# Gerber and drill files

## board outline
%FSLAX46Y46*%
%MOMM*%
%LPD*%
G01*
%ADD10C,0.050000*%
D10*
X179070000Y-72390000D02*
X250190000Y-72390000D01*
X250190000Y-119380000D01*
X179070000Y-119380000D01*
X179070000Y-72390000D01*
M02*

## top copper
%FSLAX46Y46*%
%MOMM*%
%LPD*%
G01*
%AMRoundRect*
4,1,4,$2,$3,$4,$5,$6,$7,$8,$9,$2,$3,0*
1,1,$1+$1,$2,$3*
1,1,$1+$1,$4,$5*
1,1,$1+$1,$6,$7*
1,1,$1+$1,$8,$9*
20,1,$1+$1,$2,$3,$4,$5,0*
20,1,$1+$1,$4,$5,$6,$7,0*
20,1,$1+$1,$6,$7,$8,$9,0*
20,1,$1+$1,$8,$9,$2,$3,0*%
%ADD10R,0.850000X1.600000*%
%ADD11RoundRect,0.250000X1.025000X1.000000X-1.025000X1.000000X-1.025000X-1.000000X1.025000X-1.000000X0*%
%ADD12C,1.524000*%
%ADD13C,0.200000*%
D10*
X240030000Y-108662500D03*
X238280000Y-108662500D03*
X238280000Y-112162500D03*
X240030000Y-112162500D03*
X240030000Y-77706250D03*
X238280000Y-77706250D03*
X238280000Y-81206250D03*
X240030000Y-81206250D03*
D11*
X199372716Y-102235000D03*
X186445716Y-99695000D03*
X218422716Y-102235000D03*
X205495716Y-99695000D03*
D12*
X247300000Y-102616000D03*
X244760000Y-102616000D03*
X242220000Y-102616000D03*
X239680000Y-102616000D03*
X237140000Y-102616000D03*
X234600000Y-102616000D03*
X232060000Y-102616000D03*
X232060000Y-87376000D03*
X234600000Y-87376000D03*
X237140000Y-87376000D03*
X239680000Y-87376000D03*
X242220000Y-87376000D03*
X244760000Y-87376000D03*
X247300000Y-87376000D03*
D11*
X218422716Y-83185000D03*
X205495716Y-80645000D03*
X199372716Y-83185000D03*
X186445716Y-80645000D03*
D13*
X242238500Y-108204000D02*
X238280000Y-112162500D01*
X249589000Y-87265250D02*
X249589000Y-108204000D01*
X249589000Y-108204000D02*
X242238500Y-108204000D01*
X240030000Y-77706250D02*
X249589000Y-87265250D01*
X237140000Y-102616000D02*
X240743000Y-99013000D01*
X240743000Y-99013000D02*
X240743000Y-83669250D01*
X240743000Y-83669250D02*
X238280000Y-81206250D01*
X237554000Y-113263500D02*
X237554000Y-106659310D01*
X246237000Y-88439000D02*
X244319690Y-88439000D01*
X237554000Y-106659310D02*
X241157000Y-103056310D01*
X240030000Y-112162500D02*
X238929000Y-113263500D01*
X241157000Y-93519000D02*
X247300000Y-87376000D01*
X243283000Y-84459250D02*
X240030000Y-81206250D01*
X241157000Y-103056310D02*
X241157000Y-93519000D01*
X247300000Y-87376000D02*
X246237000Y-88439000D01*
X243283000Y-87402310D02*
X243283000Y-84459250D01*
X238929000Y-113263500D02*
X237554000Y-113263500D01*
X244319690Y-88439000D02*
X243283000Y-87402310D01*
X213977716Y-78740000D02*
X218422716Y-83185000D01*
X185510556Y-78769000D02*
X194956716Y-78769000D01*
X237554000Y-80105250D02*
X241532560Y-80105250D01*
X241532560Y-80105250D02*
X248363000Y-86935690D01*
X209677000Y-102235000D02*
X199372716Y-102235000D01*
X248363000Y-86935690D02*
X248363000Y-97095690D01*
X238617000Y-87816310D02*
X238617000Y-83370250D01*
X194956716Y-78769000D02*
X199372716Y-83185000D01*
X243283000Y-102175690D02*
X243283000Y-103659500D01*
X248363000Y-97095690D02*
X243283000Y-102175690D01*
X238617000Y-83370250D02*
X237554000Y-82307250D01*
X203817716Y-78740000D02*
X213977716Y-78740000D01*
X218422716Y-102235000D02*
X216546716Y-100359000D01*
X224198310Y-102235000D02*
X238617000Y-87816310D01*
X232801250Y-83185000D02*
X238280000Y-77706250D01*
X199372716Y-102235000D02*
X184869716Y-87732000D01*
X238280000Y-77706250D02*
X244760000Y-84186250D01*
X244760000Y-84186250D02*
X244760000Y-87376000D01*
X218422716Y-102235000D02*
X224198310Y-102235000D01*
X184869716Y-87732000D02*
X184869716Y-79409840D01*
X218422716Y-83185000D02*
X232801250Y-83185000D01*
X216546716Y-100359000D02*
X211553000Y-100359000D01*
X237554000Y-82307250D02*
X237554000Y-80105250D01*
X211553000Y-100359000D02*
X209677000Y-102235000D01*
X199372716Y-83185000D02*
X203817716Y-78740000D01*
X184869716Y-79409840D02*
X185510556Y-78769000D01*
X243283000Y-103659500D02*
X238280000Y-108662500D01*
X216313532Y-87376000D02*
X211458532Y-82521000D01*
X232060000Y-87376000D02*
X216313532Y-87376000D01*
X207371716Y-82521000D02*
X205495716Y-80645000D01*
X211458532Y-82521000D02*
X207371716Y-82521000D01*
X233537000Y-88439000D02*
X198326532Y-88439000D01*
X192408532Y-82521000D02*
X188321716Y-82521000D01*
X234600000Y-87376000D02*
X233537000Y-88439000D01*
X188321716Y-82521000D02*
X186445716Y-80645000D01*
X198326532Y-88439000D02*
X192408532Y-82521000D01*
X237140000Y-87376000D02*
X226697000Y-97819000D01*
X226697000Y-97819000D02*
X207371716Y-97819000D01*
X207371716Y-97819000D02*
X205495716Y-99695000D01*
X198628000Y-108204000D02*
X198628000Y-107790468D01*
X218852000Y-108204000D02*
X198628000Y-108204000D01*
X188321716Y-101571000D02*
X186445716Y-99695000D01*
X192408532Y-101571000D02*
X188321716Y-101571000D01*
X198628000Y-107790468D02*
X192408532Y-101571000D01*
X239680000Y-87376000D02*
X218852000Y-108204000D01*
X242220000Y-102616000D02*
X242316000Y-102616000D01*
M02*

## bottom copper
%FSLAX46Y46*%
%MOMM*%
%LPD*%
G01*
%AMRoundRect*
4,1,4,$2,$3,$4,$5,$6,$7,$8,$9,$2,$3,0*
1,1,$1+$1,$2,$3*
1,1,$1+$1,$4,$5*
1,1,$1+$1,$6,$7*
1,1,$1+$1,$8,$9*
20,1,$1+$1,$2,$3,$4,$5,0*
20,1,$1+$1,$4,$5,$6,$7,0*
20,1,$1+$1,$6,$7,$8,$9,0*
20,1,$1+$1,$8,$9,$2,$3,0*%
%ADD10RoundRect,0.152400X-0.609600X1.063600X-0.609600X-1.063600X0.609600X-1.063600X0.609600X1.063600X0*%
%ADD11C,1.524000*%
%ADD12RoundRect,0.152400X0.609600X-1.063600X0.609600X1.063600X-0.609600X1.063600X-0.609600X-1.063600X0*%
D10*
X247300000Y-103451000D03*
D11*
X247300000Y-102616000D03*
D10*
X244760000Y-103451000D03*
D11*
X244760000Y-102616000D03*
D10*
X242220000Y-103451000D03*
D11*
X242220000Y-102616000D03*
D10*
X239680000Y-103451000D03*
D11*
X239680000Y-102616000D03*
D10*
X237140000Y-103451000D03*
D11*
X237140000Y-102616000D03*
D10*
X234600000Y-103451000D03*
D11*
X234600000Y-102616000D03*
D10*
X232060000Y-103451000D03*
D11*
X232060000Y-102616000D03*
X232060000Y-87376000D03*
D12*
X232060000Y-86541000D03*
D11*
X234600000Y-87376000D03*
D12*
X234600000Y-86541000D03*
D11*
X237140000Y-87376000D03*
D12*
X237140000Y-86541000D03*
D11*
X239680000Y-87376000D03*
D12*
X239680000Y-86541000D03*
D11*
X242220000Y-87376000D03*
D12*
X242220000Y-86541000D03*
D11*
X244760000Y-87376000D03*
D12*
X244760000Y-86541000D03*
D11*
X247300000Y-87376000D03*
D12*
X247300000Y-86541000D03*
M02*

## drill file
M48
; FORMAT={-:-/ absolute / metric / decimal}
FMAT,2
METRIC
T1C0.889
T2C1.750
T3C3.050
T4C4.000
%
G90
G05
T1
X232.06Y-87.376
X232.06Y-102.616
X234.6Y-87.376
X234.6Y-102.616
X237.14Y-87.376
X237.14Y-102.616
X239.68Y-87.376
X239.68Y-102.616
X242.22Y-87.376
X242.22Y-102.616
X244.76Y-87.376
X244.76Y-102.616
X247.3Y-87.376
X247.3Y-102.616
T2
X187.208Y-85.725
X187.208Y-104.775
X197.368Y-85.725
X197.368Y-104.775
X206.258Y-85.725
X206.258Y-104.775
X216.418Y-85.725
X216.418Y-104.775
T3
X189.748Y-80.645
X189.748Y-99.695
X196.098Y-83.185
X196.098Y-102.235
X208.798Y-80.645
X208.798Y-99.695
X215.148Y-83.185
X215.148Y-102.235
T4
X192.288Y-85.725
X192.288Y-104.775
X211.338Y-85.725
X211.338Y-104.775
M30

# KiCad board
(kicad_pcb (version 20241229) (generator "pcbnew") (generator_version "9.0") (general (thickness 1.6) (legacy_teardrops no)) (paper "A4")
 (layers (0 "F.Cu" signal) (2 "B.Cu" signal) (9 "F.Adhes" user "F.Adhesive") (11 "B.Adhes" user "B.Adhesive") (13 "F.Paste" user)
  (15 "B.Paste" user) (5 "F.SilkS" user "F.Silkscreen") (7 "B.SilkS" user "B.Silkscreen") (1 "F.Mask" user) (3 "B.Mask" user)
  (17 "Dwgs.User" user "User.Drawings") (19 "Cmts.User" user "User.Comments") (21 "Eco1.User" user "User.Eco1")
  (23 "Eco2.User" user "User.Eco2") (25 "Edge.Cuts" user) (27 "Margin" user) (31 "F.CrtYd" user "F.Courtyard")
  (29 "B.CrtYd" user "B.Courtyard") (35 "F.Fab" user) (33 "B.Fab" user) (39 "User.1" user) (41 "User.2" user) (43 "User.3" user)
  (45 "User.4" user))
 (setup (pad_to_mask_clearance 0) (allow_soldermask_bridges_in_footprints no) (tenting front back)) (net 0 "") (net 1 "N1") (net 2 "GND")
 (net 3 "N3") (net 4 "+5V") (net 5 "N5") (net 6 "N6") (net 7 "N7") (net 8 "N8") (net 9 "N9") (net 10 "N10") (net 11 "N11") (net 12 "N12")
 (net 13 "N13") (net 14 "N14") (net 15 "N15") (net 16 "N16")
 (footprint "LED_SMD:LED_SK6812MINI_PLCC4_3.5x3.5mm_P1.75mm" (layer "F.Cu") (at 239.155 110.4125 -90)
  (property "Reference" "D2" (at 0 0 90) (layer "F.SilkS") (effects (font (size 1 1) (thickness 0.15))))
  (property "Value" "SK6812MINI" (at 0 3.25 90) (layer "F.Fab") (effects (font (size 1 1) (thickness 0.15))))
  (pad "1" smd rect (at -1.75 -0.875 270) (size 1.6 0.85) (layers "F.Cu" "F.Mask" "F.Paste") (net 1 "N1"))
  (pad "2" smd rect (at -1.75 0.875 270) (size 1.6 0.85) (layers "F.Cu" "F.Mask" "F.Paste") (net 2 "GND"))
  (pad "3" smd rect (at 1.75 0.875 270) (size 1.6 0.85) (layers "F.Cu" "F.Mask" "F.Paste") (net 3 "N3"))
  (pad "4" smd rect (at 1.75 -0.875 270) (size 1.6 0.85) (layers "F.Cu" "F.Mask" "F.Paste") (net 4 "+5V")))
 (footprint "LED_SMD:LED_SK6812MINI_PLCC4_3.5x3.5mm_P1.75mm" (layer "F.Cu") (at 239.155 79.45625 -90)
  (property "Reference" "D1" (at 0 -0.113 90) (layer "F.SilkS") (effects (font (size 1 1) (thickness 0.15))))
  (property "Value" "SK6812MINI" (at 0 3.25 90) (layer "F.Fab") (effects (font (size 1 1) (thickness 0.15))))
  (pad "1" smd rect (at -1.75 -0.875 270) (size 1.6 0.85) (layers "F.Cu" "F.Mask" "F.Paste") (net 3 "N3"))
  (pad "2" smd rect (at -1.75 0.875 270) (size 1.6 0.85) (layers "F.Cu" "F.Mask" "F.Paste") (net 2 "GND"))
  (pad "3" smd rect (at 1.75 0.875 270) (size 1.6 0.85) (layers "F.Cu" "F.Mask" "F.Paste") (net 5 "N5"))
  (pad "4" smd rect (at 1.75 -0.875 270) (size 1.6 0.85) (layers "F.Cu" "F.Mask" "F.Paste") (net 4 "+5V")))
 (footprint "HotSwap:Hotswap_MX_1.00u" (layer "B.Cu") (at 192.287716 104.775 180)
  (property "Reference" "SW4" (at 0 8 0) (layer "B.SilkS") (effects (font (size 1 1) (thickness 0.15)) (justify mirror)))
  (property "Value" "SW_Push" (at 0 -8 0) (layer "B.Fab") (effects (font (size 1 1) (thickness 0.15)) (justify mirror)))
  (pad "" np_thru_hole circle (at -5.08 0 180) (size 1.75 1.75) (drill 1.75) (layers "*.Cu" "*.Mask"))
  (pad "" np_thru_hole circle (at -3.81 2.54 180) (size 3.05 3.05) (drill 3.05) (layers "*.Cu" "*.Mask"))
  (pad "" np_thru_hole circle (at 0 0 180) (size 4 4) (drill 4) (layers "*.Cu" "*.Mask"))
  (pad "" np_thru_hole circle (at 2.54 5.08 180) (size 3.05 3.05) (drill 3.05) (layers "*.Cu" "*.Mask"))
  (pad "" np_thru_hole circle (at 5.08 0 180) (size 1.75 1.75) (drill 1.75) (layers "*.Cu" "*.Mask"))
  (pad "1" smd roundrect (at -7.085 2.54 180) (size 2.55 2.5) (layers "F.Cu" "F.Mask" "F.Paste") (roundrect_rratio 0.1) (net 2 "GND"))
  (pad "2" smd roundrect (at 5.842 5.08 180) (size 2.55 2.5) (layers "F.Cu" "F.Mask" "F.Paste") (roundrect_rratio 0.1) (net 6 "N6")))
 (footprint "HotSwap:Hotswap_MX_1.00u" (layer "B.Cu") (at 211.337716 104.775 180)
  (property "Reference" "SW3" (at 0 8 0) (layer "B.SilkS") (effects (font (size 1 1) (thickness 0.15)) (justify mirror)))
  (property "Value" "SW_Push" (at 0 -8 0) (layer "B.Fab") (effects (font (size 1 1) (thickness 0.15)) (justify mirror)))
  (pad "" np_thru_hole circle (at -5.08 0 180) (size 1.75 1.75) (drill 1.75) (layers "*.Cu" "*.Mask"))
  (pad "" np_thru_hole circle (at -3.81 2.54 180) (size 3.05 3.05) (drill 3.05) (layers "*.Cu" "*.Mask"))
  (pad "" np_thru_hole circle (at 0 0 180) (size 4 4) (drill 4) (layers "*.Cu" "*.Mask"))
  (pad "" np_thru_hole circle (at 2.54 5.08 180) (size 3.05 3.05) (drill 3.05) (layers "*.Cu" "*.Mask"))
  (pad "" np_thru_hole circle (at 5.08 0 180) (size 1.75 1.75) (drill 1.75) (layers "*.Cu" "*.Mask"))
  (pad "1" smd roundrect (at -7.085 2.54 180) (size 2.55 2.5) (layers "F.Cu" "F.Mask" "F.Paste") (roundrect_rratio 0.1) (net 2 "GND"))
  (pad "2" smd roundrect (at 5.842 5.08 180) (size 2.55 2.5) (layers "F.Cu" "F.Mask" "F.Paste") (roundrect_rratio 0.1) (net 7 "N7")))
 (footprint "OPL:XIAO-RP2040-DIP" (layer "B.Cu") (at 239.68 94.996 90)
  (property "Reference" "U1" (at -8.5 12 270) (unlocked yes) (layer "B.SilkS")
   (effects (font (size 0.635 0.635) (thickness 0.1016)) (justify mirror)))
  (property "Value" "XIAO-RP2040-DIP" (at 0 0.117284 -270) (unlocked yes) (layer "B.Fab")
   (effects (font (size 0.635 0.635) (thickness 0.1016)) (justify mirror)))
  (pad "1" smd roundrect (at -8.455 7.62 270) (size 2.432 1.524) (layers "B.Cu" "B.Mask") (roundrect_rratio 0.1) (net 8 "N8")
   (thermal_bridge_angle 45))
  (pad "1" thru_hole circle (at -7.62 7.62 270) (size 1.524 1.524) (drill 0.889) (layers "*.Cu" "*.Mask") (remove_unused_layers no)
   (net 8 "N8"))
  (pad "2" smd roundrect (at -8.455 5.08 270) (size 2.432 1.524) (layers "B.Cu" "B.Mask") (roundrect_rratio 0.1) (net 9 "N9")
   (thermal_bridge_angle 45))
  (pad "2" thru_hole circle (at -7.62 5.08 270) (size 1.524 1.524) (drill 0.889) (layers "*.Cu" "*.Mask") (remove_unused_layers no)
   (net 9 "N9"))
  (pad "3" smd roundrect (at -8.455 2.54 270) (size 2.432 1.524) (layers "B.Cu" "B.Mask") (roundrect_rratio 0.1) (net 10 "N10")
   (thermal_bridge_angle 45))
  (pad "3" thru_hole circle (at -7.62 2.54 270) (size 1.524 1.524) (drill 0.889) (layers "*.Cu" "*.Mask") (remove_unused_layers no)
   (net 10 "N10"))
  (pad "4" smd roundrect (at -8.455 0 270) (size 2.432 1.524) (layers "B.Cu" "B.Mask") (roundrect_rratio 0.1) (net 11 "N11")
   (thermal_bridge_angle 45))
  (pad "4" thru_hole circle (at -7.62 0 270) (size 1.524 1.524) (drill 0.889) (layers "*.Cu" "*.Mask") (remove_unused_layers no)
   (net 11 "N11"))
  (pad "5" smd roundrect (at -8.455 -2.54 270) (size 2.432 1.524) (layers "B.Cu" "B.Mask") (roundrect_rratio 0.1) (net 5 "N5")
   (thermal_bridge_angle 45))
  (pad "5" thru_hole circle (at -7.62 -2.54 270) (size 1.524 1.524) (drill 0.889) (layers "*.Cu" "*.Mask") (remove_unused_layers no)
   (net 5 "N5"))
  (pad "6" smd roundrect (at -8.455 -5.08 270) (size 2.432 1.524) (layers "B.Cu" "B.Mask") (roundrect_rratio 0.1) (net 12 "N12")
   (thermal_bridge_angle 45))
  (pad "6" thru_hole circle (at -7.62 -5.08 270) (size 1.524 1.524) (drill 0.889) (layers "*.Cu" "*.Mask") (remove_unused_layers no)
   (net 12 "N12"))
  (pad "7" smd roundrect (at -8.455 -7.62 270) (size 2.432 1.524) (layers "B.Cu" "B.Mask") (roundrect_rratio 0.1) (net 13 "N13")
   (thermal_bridge_angle 45))
  (pad "7" thru_hole circle (at -7.62 -7.62 270) (size 1.524 1.524) (drill 0.889) (layers "*.Cu" "*.Mask") (remove_unused_layers no)
   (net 13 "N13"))
  (pad "8" thru_hole circle (at 7.62 -7.62 90) (size 1.524 1.524) (drill 0.889) (layers "*.Cu" "*.Mask") (remove_unused_layers no)
   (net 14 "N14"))
  (pad "8" smd roundrect (at 8.455 -7.62 90) (size 2.432 1.524) (layers "B.Cu" "B.Mask") (roundrect_rratio 0.1) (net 14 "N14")
   (thermal_bridge_angle 45))
  (pad "9" thru_hole circle (at 7.62 -5.08 90) (size 1.524 1.524) (drill 0.889) (layers "*.Cu" "*.Mask") (remove_unused_layers no)
   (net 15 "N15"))
  (pad "9" smd roundrect (at 8.455 -5.08 90) (size 2.432 1.524) (layers "B.Cu" "B.Mask") (roundrect_rratio 0.1) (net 15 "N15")
   (thermal_bridge_angle 45))
  (pad "10" thru_hole circle (at 7.62 -2.54 90) (size 1.524 1.524) (drill 0.889) (layers "*.Cu" "*.Mask") (remove_unused_layers no)
   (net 7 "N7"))
  (pad "10" smd roundrect (at 8.455 -2.54 90) (size 2.432 1.524) (layers "B.Cu" "B.Mask") (roundrect_rratio 0.1) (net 7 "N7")
   (thermal_bridge_angle 45))
  (pad "11" thru_hole circle (at 7.62 0 90) (size 1.524 1.524) (drill 0.889) (layers "*.Cu" "*.Mask") (remove_unused_layers no) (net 6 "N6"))
  (pad "11" smd roundrect (at 8.455 0 90) (size 2.432 1.524) (layers "B.Cu" "B.Mask") (roundrect_rratio 0.1) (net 6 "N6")
   (thermal_bridge_angle 45))
  (pad "12" thru_hole circle (at 7.62 2.54 90) (size 1.524 1.524) (drill 0.889) (layers "*.Cu" "*.Mask") (remove_unused_layers no)
   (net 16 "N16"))
  (pad "12" smd roundrect (at 8.455 2.54 90) (size 2.432 1.524) (layers "B.Cu" "B.Mask") (roundrect_rratio 0.1) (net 16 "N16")
   (thermal_bridge_angle 45))
  (pad "13" thru_hole circle (at 7.62 5.08 90) (size 1.524 1.524) (drill 0.889) (layers "*.Cu" "*.Mask") (remove_unused_layers no)
   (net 2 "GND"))
  (pad "13" smd roundrect (at 8.455 5.08 90) (size 2.432 1.524) (layers "B.Cu" "B.Mask") (roundrect_rratio 0.1) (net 2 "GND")
   (thermal_bridge_angle 45))
  (pad "14" thru_hole circle (at 7.62 7.62 90) (size 1.524 1.524) (drill 0.889) (layers "*.Cu" "*.Mask") (remove_unused_layers no)
   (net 4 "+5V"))
  (pad "14" smd roundrect (at 8.455 7.62 90) (size 2.432 1.524) (layers "B.Cu" "B.Mask") (roundrect_rratio 0.1) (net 4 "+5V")
   (thermal_bridge_angle 45)))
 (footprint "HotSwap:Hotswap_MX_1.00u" (layer "B.Cu") (at 211.337716 85.725 180)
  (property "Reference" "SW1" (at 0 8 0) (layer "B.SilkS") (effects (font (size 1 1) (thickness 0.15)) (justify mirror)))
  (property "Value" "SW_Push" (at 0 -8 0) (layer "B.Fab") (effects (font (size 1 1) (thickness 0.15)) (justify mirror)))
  (pad "" np_thru_hole circle (at -5.08 0 180) (size 1.75 1.75) (drill 1.75) (layers "*.Cu" "*.Mask"))
  (pad "" np_thru_hole circle (at -3.81 2.54 180) (size 3.05 3.05) (drill 3.05) (layers "*.Cu" "*.Mask"))
  (pad "" np_thru_hole circle (at 0 0 180) (size 4 4) (drill 4) (layers "*.Cu" "*.Mask"))
  (pad "" np_thru_hole circle (at 2.54 5.08 180) (size 3.05 3.05) (drill 3.05) (layers "*.Cu" "*.Mask"))
  (pad "" np_thru_hole circle (at 5.08 0 180) (size 1.75 1.75) (drill 1.75) (layers "*.Cu" "*.Mask"))
  (pad "1" smd roundrect (at -7.085 2.54 180) (size 2.55 2.5) (layers "F.Cu" "F.Mask" "F.Paste") (roundrect_rratio 0.1) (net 2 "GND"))
  (pad "2" smd roundrect (at 5.842 5.08 180) (size 2.55 2.5) (layers "F.Cu" "F.Mask" "F.Paste") (roundrect_rratio 0.1) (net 14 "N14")))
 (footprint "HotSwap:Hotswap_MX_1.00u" (layer "B.Cu") (at 192.287716 85.725 180)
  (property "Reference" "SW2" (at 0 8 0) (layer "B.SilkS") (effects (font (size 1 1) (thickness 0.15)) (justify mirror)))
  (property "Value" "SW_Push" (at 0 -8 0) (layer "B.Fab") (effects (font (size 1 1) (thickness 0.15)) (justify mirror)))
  (pad "" np_thru_hole circle (at -5.08 0 180) (size 1.75 1.75) (drill 1.75) (layers "*.Cu" "*.Mask"))
  (pad "" np_thru_hole circle (at -3.81 2.54 180) (size 3.05 3.05) (drill 3.05) (layers "*.Cu" "*.Mask"))
  (pad "" np_thru_hole circle (at 0 0 180) (size 4 4) (drill 4) (layers "*.Cu" "*.Mask"))
  (pad "" np_thru_hole circle (at 2.54 5.08 180) (size 3.05 3.05) (drill 3.05) (layers "*.Cu" "*.Mask"))
  (pad "" np_thru_hole circle (at 5.08 0 180) (size 1.75 1.75) (drill 1.75) (layers "*.Cu" "*.Mask"))
  (pad "1" smd roundrect (at -7.085 2.54 180) (size 2.55 2.5) (layers "F.Cu" "F.Mask" "F.Paste") (roundrect_rratio 0.1) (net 2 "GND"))
  (pad "2" smd roundrect (at 5.842 5.08 180) (size 2.55 2.5) (layers "F.Cu" "F.Mask" "F.Paste") (roundrect_rratio 0.1) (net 15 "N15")))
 (gr_rect (start 179.07 72.39) (end 250.19 119.38) (stroke (width 0.05) (type default)) (fill no) (layer "Edge.Cuts"))
 (segment (start 242.2385 108.204) (end 238.28 112.1625) (width 0.2) (layer "F.Cu") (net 3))
 (segment (start 249.589 87.26525) (end 249.589 108.204) (width 0.2) (layer "F.Cu") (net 3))
 (segment (start 249.589 108.204) (end 242.2385 108.204) (width 0.2) (layer "F.Cu") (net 3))
 (segment (start 240.03 77.70625) (end 249.589 87.26525) (width 0.2) (layer "F.Cu") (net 3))
 (segment (start 237.14 102.616) (end 240.743 99.013) (width 0.2) (layer "F.Cu") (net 5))
 (segment (start 240.743 99.013) (end 240.743 83.66925) (width 0.2) (layer "F.Cu") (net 5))
 (segment (start 240.743 83.66925) (end 238.28 81.20625) (width 0.2) (layer "F.Cu") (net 5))
 (segment (start 237.554 113.2635) (end 237.554 106.65931) (width 0.2) (layer "F.Cu") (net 4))
 (segment (start 246.237 88.439) (end 244.31969 88.439) (width 0.2) (layer "F.Cu") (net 4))
 (segment (start 237.554 106.65931) (end 241.157 103.05631) (width 0.2) (layer "F.Cu") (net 4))
 (segment (start 240.03 112.1625) (end 238.929 113.2635) (width 0.2) (layer "F.Cu") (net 4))
 (segment (start 241.157 93.519) (end 247.3 87.376) (width 0.2) (layer "F.Cu") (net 4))
 (segment (start 243.283 84.45925) (end 240.03 81.20625) (width 0.2) (layer "F.Cu") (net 4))
 (segment (start 241.157 103.05631) (end 241.157 93.519) (width 0.2) (layer "F.Cu") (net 4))
 (segment (start 247.3 87.376) (end 246.237 88.439) (width 0.2) (layer "F.Cu") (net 4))
 (segment (start 243.283 87.40231) (end 243.283 84.45925) (width 0.2) (layer "F.Cu") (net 4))
 (segment (start 238.929 113.2635) (end 237.554 113.2635) (width 0.2) (layer "F.Cu") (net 4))
 (segment (start 244.31969 88.439) (end 243.283 87.40231) (width 0.2) (layer "F.Cu") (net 4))
 (segment (start 213.977716 78.74) (end 218.422716 83.185) (width 0.2) (layer "F.Cu") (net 2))
 (segment (start 185.510556 78.769) (end 194.956716 78.769) (width 0.2) (layer "F.Cu") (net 2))
 (segment (start 237.554 80.10525) (end 241.53256 80.10525) (width 0.2) (layer "F.Cu") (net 2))
 (segment (start 241.53256 80.10525) (end 248.363 86.93569) (width 0.2) (layer "F.Cu") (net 2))
 (segment (start 209.677 102.235) (end 199.372716 102.235) (width 0.2) (layer "F.Cu") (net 2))
 (segment (start 248.363 86.93569) (end 248.363 97.09569) (width 0.2) (layer "F.Cu") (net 2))
 (segment (start 238.617 87.81631) (end 238.617 83.37025) (width 0.2) (layer "F.Cu") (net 2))
 (segment (start 194.956716 78.769) (end 199.372716 83.185) (width 0.2) (layer "F.Cu") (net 2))
 (segment (start 243.283 102.17569) (end 243.283 103.6595) (width 0.2) (layer "F.Cu") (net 2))
 (segment (start 248.363 97.09569) (end 243.283 102.17569) (width 0.2) (layer "F.Cu") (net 2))
 (segment (start 238.617 83.37025) (end 237.554 82.30725) (width 0.2) (layer "F.Cu") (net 2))
 (segment (start 203.817716 78.74) (end 213.977716 78.74) (width 0.2) (layer "F.Cu") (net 2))
 (segment (start 218.422716 102.235) (end 216.546716 100.359) (width 0.2) (layer "F.Cu") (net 2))
 (segment (start 224.19831 102.235) (end 238.617 87.81631) (width 0.2) (layer "F.Cu") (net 2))
 (segment (start 232.80125 83.185) (end 238.28 77.70625) (width 0.2) (layer "F.Cu") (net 2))
 (segment (start 199.372716 102.235) (end 184.869716 87.732) (width 0.2) (layer "F.Cu") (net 2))
 (segment (start 238.28 77.70625) (end 244.76 84.18625) (width 0.2) (layer "F.Cu") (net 2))
 (segment (start 244.76 84.18625) (end 244.76 87.376) (width 0.2) (layer "F.Cu") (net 2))
 (segment (start 218.422716 102.235) (end 224.19831 102.235) (width 0.2) (layer "F.Cu") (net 2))
 (segment (start 184.869716 87.732) (end 184.869716 79.40984) (width 0.2) (layer "F.Cu") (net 2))
 (segment (start 218.422716 83.185) (end 232.80125 83.185) (width 0.2) (layer "F.Cu") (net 2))
 (segment (start 216.546716 100.359) (end 211.553 100.359) (width 0.2) (layer "F.Cu") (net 2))
 (segment (start 237.554 82.30725) (end 237.554 80.10525) (width 0.2) (layer "F.Cu") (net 2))
 (segment (start 211.553 100.359) (end 209.677 102.235) (width 0.2) (layer "F.Cu") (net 2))
 (segment (start 199.372716 83.185) (end 203.817716 78.74) (width 0.2) (layer "F.Cu") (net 2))
 (segment (start 184.869716 79.40984) (end 185.510556 78.769) (width 0.2) (layer "F.Cu") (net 2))
 (segment (start 243.283 103.6595) (end 238.28 108.6625) (width 0.2) (layer "F.Cu") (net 2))
 (segment (start 216.313532 87.376) (end 211.458532 82.521) (width 0.2) (layer "F.Cu") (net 14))
 (segment (start 232.06 87.376) (end 216.313532 87.376) (width 0.2) (layer "F.Cu") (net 14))
 (segment (start 207.371716 82.521) (end 205.495716 80.645) (width 0.2) (layer "F.Cu") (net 14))
 (segment (start 211.458532 82.521) (end 207.371716 82.521) (width 0.2) (layer "F.Cu") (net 14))
 (segment (start 233.537 88.439) (end 198.326532 88.439) (width 0.2) (layer "F.Cu") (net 15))
 (segment (start 192.408532 82.521) (end 188.321716 82.521) (width 0.2) (layer "F.Cu") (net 15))
 (segment (start 234.6 87.376) (end 233.537 88.439) (width 0.2) (layer "F.Cu") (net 15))
 (segment (start 188.321716 82.521) (end 186.445716 80.645) (width 0.2) (layer "F.Cu") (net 15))
 (segment (start 198.326532 88.439) (end 192.408532 82.521) (width 0.2) (layer "F.Cu") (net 15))
 (segment (start 237.14 87.376) (end 226.697 97.819) (width 0.2) (layer "F.Cu") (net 7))
 (segment (start 226.697 97.819) (end 207.371716 97.819) (width 0.2) (layer "F.Cu") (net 7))
 (segment (start 207.371716 97.819) (end 205.495716 99.695) (width 0.2) (layer "F.Cu") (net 7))
 (segment (start 198.628 108.204) (end 198.628 107.790468) (width 0.2) (layer "F.Cu") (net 6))
 (segment (start 218.852 108.204) (end 198.628 108.204) (width 0.2) (layer "F.Cu") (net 6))
 (segment (start 188.321716 101.571) (end 186.445716 99.695) (width 0.2) (layer "F.Cu") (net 6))
 (segment (start 192.408532 101.571) (end 188.321716 101.571) (width 0.2) (layer "F.Cu") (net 6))
 (segment (start 198.628 107.790468) (end 192.408532 101.571) (width 0.2) (layer "F.Cu") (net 6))
 (segment (start 239.68 87.376) (end 218.852 108.204) (width 0.2) (layer "F.Cu") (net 6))
 (segment (start 242.22 102.616) (end 242.316 102.616) (width 0.2) (layer "F.Cu") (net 10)))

